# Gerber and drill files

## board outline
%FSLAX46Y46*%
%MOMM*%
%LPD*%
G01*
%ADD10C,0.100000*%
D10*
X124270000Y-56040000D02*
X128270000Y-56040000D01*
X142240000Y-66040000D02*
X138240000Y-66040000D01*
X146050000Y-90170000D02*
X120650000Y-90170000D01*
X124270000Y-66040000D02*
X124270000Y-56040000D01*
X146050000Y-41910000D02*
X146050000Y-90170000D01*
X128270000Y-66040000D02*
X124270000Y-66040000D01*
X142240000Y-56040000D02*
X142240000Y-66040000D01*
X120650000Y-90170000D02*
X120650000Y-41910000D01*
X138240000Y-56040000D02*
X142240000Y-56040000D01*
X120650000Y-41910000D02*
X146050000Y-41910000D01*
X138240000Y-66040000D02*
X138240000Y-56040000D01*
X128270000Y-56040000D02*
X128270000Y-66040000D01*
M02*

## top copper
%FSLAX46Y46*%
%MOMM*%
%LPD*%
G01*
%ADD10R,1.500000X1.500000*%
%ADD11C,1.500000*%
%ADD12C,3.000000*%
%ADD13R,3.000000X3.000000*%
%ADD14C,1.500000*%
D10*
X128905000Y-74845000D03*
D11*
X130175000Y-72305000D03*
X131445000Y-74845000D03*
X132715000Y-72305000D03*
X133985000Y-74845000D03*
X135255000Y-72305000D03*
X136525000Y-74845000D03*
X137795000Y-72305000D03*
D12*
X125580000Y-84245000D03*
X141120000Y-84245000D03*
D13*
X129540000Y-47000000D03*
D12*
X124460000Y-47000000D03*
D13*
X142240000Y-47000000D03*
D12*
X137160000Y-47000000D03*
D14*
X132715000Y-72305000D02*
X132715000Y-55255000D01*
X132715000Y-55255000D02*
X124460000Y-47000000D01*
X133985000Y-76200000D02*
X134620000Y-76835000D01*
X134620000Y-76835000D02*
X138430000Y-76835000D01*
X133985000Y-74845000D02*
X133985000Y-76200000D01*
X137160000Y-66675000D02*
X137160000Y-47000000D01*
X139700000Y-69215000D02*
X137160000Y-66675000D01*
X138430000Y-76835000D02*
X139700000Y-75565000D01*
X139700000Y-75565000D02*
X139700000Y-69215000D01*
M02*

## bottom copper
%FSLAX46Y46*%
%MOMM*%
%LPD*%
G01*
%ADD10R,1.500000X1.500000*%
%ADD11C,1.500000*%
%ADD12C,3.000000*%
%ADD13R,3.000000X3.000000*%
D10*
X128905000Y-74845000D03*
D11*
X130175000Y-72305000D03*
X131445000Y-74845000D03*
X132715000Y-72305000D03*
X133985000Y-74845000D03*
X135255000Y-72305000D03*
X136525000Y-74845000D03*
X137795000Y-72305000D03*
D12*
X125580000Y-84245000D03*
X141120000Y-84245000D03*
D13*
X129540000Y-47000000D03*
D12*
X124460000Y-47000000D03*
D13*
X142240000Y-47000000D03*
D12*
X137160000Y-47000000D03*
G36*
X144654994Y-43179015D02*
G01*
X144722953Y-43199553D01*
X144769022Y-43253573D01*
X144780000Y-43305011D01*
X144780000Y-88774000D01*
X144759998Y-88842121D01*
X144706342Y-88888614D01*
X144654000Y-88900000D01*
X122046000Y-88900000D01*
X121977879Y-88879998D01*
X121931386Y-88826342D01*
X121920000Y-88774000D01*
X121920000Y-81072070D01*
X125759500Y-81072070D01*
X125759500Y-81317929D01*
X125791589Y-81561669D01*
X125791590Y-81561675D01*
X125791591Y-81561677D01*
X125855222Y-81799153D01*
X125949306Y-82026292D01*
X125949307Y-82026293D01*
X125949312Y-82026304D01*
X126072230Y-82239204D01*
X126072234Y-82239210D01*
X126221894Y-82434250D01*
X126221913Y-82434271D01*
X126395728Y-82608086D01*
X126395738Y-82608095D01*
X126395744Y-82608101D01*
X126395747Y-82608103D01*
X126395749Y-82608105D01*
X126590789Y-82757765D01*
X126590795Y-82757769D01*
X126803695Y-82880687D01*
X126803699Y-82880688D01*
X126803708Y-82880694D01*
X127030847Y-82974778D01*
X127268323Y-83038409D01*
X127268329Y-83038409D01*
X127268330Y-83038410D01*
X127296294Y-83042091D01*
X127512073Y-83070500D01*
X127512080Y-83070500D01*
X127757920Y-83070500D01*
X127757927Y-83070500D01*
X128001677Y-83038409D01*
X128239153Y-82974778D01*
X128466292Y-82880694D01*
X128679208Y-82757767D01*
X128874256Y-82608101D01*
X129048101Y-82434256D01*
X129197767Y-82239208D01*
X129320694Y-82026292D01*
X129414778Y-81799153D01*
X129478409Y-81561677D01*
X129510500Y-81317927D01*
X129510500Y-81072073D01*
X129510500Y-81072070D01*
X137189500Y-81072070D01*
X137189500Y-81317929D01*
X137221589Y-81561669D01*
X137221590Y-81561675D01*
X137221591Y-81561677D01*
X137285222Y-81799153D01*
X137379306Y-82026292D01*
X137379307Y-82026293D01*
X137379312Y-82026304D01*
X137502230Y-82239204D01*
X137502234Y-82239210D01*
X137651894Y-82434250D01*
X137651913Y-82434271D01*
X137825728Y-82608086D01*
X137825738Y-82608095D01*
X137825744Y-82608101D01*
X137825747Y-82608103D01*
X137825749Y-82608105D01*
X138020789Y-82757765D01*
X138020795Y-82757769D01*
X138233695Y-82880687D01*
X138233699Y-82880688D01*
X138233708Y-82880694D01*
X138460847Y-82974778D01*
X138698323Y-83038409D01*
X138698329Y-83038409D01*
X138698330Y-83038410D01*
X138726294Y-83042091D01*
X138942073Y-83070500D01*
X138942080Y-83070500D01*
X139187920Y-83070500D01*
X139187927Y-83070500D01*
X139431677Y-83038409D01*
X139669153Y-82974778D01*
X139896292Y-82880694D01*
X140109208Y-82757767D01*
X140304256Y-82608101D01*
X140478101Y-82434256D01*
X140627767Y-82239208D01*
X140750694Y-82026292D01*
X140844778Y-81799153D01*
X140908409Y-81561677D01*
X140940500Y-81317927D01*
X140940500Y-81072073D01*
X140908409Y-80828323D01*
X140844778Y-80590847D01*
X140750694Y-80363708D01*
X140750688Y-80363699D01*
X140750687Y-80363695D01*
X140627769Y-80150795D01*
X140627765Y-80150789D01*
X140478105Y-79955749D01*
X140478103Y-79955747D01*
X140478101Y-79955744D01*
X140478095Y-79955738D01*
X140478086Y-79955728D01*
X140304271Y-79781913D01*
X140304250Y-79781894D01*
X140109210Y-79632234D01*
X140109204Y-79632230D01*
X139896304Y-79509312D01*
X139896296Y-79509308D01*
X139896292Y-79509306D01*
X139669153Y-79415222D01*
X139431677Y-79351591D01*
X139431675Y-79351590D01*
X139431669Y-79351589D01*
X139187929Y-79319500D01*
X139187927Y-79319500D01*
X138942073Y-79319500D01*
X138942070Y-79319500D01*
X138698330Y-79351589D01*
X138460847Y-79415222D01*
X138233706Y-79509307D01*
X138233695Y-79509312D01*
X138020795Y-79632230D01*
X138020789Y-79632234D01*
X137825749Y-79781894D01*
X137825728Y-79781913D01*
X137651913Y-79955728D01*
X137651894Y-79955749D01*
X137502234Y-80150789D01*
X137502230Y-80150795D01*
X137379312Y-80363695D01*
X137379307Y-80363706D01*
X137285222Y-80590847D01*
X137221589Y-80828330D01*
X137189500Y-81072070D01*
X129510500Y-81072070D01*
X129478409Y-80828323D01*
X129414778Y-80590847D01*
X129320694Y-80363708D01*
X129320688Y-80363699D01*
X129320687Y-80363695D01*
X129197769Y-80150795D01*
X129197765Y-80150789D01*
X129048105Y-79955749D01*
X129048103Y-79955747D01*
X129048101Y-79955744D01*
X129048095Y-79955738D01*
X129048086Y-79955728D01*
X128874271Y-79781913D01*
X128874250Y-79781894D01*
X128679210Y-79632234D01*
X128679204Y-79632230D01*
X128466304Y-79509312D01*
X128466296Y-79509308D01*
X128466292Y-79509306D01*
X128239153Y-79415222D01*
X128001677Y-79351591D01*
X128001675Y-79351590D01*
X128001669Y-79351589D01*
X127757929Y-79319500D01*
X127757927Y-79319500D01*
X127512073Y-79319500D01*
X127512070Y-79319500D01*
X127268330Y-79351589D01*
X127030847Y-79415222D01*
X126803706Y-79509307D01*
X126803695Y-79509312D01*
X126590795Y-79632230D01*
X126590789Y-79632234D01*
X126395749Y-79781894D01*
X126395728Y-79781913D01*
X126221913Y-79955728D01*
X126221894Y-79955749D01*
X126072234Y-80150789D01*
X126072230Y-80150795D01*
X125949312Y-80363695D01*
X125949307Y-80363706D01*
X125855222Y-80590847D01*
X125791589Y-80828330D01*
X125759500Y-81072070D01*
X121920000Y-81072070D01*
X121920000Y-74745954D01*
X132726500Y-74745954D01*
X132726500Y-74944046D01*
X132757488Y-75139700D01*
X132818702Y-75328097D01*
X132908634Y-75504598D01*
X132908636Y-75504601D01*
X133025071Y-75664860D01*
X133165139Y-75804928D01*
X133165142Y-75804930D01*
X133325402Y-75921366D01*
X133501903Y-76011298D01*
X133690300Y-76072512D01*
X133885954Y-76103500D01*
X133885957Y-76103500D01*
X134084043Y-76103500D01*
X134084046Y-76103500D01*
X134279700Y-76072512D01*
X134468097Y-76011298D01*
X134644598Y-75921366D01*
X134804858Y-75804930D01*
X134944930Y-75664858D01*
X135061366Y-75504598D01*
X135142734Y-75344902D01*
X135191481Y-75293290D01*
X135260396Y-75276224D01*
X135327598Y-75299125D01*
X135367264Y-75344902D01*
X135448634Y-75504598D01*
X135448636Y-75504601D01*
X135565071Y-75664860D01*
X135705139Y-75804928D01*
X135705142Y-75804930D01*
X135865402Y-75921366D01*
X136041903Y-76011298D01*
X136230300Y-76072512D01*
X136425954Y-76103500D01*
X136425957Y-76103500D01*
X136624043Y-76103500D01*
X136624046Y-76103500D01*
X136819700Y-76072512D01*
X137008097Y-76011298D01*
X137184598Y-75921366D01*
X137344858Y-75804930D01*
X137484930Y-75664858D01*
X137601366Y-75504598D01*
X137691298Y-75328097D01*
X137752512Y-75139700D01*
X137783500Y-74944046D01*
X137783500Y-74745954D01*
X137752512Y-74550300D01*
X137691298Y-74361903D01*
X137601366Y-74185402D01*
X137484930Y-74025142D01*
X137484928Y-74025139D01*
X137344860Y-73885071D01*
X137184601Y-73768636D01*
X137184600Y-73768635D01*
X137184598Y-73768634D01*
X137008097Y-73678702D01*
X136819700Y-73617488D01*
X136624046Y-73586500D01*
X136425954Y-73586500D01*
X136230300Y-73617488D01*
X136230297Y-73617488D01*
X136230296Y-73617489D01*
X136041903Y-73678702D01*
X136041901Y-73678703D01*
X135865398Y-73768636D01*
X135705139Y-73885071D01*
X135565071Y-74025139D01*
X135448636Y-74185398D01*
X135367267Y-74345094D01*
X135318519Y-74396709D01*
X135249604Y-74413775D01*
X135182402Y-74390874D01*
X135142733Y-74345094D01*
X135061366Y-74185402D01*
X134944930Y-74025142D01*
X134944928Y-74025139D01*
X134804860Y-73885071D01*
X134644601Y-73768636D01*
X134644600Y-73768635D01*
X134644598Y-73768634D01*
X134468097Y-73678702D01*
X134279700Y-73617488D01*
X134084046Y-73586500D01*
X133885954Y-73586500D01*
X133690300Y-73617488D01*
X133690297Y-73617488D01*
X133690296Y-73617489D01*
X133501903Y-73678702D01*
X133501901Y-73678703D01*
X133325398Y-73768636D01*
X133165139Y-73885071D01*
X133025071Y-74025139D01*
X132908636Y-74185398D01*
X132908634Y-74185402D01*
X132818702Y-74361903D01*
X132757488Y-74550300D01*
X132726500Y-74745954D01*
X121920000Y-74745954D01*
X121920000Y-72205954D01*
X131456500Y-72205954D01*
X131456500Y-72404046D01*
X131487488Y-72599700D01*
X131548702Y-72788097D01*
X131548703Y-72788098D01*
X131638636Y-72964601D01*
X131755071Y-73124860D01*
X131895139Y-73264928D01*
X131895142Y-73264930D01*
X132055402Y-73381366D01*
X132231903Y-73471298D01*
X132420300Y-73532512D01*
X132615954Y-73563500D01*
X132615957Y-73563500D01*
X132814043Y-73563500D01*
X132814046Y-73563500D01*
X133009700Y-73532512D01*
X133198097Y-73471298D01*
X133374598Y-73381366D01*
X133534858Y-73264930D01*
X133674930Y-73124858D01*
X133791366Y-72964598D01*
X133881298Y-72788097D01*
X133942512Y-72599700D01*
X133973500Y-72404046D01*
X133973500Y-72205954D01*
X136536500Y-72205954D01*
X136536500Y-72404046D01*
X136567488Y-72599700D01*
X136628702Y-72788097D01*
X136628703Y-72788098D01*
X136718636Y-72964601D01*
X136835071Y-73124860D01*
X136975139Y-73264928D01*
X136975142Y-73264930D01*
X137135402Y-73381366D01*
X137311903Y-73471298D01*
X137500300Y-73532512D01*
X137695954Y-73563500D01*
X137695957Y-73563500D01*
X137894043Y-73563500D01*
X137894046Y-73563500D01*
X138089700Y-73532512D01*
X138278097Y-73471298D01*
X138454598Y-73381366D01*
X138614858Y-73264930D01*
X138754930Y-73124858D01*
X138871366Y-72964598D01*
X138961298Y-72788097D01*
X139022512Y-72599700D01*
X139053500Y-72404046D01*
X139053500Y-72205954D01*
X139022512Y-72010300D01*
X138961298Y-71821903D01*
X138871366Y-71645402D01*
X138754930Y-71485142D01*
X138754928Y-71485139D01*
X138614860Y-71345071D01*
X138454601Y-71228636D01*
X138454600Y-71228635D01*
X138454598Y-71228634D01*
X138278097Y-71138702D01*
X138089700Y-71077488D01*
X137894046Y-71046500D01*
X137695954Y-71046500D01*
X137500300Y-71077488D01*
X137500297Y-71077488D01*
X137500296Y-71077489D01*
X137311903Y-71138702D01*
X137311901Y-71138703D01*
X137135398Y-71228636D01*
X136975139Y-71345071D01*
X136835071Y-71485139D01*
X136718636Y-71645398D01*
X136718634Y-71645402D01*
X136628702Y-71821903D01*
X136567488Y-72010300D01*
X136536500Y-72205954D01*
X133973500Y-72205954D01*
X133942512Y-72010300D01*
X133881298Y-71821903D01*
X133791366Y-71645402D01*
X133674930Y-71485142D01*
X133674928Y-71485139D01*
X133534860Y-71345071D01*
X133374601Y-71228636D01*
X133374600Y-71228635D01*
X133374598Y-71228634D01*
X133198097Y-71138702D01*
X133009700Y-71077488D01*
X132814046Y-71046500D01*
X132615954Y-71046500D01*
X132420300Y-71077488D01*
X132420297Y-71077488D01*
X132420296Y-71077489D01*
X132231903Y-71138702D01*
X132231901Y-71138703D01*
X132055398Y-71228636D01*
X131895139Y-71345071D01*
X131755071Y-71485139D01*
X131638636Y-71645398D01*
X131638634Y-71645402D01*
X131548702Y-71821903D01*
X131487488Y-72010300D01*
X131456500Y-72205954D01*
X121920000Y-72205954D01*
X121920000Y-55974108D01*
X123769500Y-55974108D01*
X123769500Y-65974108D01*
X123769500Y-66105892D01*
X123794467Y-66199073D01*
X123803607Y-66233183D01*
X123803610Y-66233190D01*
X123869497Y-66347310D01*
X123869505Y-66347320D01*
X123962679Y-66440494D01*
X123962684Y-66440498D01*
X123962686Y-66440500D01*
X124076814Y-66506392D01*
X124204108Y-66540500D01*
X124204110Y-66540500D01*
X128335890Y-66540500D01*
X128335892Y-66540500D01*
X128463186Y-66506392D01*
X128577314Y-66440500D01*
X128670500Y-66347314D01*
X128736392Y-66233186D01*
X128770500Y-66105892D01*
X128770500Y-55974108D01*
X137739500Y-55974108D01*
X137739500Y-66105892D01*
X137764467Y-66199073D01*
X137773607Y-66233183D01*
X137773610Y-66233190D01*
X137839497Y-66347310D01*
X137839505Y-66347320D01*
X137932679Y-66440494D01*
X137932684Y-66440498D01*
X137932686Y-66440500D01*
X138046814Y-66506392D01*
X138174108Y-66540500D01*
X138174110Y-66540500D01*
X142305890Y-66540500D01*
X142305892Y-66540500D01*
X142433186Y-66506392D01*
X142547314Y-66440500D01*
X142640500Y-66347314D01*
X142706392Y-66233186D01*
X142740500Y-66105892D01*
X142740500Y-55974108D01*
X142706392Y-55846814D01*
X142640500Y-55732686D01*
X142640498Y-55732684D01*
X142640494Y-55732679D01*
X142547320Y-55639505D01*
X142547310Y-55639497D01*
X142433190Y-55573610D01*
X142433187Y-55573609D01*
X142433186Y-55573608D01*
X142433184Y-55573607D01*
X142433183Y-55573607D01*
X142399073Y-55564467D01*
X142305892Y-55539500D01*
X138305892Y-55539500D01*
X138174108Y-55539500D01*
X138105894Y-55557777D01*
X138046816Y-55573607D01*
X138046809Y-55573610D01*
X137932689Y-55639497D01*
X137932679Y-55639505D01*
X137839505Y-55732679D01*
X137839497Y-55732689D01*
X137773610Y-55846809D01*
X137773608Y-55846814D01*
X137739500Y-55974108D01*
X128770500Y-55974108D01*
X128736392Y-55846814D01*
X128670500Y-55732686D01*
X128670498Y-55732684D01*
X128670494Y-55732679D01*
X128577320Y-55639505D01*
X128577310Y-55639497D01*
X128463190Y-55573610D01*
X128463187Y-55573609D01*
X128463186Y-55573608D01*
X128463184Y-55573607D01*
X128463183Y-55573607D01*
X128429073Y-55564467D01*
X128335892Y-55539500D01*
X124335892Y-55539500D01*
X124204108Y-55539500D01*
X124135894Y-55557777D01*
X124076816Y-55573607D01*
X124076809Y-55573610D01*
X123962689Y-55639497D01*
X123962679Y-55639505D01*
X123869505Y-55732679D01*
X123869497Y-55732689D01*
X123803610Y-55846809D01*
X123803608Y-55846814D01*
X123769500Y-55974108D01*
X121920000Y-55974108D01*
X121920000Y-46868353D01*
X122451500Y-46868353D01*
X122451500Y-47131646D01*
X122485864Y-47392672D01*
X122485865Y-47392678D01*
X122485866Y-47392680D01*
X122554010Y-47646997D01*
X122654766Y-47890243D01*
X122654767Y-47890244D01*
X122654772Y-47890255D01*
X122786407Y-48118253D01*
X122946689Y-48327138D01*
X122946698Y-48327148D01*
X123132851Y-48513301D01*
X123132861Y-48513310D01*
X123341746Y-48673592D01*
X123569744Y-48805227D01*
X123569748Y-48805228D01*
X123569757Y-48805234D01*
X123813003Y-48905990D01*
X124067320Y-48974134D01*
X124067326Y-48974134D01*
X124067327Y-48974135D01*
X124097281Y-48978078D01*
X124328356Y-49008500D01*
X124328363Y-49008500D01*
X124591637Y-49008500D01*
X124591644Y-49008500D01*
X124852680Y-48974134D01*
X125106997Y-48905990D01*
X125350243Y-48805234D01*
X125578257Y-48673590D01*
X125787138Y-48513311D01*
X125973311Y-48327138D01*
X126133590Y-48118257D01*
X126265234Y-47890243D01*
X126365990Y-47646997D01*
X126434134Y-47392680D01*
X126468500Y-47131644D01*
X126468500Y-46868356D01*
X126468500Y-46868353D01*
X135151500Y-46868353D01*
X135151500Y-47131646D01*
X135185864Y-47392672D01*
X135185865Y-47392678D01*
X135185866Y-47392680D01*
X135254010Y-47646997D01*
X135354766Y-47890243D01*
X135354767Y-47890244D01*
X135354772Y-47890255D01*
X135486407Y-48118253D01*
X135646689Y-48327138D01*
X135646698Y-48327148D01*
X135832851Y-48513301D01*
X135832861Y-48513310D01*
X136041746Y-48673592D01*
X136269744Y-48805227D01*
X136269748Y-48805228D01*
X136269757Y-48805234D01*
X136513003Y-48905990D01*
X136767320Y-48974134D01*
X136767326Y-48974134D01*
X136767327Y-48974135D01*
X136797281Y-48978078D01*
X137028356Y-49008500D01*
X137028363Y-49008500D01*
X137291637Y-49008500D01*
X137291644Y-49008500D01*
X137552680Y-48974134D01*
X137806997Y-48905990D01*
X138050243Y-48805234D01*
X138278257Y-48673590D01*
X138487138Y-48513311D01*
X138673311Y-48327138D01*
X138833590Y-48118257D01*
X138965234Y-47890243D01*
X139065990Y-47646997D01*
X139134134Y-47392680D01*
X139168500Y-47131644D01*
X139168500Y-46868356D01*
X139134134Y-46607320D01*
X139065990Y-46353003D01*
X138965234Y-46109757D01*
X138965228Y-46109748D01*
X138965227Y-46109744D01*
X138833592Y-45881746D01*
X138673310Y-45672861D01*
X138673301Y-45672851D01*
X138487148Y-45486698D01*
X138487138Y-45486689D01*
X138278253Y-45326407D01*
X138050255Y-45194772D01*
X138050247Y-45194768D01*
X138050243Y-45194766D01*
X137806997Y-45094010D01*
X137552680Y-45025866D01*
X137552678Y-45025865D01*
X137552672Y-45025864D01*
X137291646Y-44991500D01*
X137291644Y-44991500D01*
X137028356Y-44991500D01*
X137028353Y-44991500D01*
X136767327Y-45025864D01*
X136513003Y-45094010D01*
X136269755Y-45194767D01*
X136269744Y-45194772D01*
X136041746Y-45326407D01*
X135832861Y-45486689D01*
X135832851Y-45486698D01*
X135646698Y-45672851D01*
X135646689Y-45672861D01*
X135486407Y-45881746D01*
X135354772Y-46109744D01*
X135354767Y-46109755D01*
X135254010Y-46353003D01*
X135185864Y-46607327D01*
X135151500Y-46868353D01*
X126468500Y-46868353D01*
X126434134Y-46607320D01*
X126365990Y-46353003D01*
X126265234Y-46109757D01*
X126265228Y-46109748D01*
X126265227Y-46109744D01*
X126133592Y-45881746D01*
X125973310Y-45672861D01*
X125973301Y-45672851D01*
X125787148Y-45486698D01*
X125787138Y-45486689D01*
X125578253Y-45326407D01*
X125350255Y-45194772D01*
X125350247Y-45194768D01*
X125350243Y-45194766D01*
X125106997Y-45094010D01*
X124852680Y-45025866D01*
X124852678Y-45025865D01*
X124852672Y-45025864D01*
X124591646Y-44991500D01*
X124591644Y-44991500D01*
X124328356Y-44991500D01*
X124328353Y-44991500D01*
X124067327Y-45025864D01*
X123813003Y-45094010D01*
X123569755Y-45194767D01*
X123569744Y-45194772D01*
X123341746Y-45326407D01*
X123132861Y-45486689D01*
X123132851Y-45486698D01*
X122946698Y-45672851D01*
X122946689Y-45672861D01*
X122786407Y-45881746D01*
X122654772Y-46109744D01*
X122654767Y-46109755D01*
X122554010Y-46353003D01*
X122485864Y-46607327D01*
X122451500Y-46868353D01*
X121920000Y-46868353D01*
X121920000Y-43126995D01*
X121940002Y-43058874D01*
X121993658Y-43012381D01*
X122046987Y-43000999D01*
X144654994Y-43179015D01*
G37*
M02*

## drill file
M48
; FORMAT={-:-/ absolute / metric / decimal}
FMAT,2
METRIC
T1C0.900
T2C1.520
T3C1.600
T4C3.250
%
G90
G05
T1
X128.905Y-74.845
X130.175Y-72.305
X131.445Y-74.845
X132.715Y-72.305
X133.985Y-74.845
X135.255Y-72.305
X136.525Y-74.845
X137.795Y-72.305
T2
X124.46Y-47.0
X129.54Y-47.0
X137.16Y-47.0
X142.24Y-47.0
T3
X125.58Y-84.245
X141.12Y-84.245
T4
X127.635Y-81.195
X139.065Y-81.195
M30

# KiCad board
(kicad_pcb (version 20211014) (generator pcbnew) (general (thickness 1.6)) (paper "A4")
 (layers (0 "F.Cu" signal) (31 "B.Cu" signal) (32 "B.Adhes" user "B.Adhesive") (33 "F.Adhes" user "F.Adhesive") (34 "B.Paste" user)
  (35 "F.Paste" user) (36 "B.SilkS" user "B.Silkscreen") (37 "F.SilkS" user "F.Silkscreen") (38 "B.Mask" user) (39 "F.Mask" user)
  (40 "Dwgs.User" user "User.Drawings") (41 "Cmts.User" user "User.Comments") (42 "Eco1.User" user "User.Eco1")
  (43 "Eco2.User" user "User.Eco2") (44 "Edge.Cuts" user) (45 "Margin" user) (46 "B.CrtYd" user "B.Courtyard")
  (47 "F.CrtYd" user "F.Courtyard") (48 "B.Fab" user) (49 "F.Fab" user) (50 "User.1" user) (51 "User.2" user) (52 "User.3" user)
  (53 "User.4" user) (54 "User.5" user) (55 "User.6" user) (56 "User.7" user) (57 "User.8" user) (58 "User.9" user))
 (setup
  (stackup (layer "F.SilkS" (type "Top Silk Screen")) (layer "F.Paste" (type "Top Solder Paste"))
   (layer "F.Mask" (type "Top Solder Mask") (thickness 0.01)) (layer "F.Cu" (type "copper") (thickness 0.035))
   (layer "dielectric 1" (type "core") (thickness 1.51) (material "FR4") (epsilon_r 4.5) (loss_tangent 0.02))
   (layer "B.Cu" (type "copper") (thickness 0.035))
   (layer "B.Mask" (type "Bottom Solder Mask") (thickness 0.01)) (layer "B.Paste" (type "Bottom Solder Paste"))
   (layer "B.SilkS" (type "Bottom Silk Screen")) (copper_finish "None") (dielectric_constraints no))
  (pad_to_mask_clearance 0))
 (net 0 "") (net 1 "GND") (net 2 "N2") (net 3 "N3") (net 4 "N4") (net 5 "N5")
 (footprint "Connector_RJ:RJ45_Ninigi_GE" (layer "F.Cu") (at 128.905 74.845)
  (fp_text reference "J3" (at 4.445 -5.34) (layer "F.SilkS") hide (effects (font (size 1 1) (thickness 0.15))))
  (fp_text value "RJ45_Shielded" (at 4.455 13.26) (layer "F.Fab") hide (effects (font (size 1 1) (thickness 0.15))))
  (pad "" np_thru_hole circle (at -1.27 6.35) (size 3.25 3.25) (drill 3.25) (layers *.Cu *.Mask))
  (pad "" np_thru_hole circle (at 10.16 6.35 180) (size 3.25 3.25) (drill 3.25) (layers *.Cu *.Mask))
  (pad "1" thru_hole rect (at 0 0 180) (size 1.5 1.5) (drill 0.9) (layers *.Cu *.Mask) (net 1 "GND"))
  (pad "2" thru_hole circle (at 1.27 -2.54 180) (size 1.5 1.5) (drill 0.9) (layers *.Cu *.Mask) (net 1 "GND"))
  (pad "3" thru_hole circle (at 2.54 0 180) (size 1.5 1.5) (drill 0.9) (layers *.Cu *.Mask) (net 1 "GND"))
  (pad "4" thru_hole circle (at 3.81 -2.54 180) (size 1.5 1.5) (drill 0.9) (layers *.Cu *.Mask) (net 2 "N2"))
  (pad "5" thru_hole circle (at 5.08 0 180) (size 1.5 1.5) (drill 0.9) (layers *.Cu *.Mask) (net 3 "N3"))
  (pad "6" thru_hole circle (at 6.35 -2.54 180) (size 1.5 1.5) (drill 0.9) (layers *.Cu *.Mask) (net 1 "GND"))
  (pad "7" thru_hole circle (at 7.62 0 180) (size 1.5 1.5) (drill 0.9) (layers *.Cu *.Mask) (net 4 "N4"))
  (pad "8" thru_hole circle (at 8.89 -2.54 180) (size 1.5 1.5) (drill 0.9) (layers *.Cu *.Mask) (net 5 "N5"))
  (pad "SH" thru_hole circle (at -3.325 9.4) (size 3 3) (drill 1.6) (layers *.Cu *.Mask) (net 1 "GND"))
  (pad "SH" thru_hole circle (at 12.215 9.4 180) (size 3 3) (drill 1.6) (layers *.Cu *.Mask) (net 1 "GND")))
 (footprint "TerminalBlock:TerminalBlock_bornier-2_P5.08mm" (layer "F.Cu") (at 129.54 47 180)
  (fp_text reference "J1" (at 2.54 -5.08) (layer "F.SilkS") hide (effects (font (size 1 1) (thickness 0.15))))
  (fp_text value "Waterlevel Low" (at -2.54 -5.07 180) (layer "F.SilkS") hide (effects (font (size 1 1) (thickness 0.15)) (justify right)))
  (pad "1" thru_hole rect (at 0 0 180) (size 3 3) (drill 1.52) (layers *.Cu *.Mask) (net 1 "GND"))
  (pad "2" thru_hole circle (at 5.08 0 180) (size 3 3) (drill 1.52) (layers *.Cu *.Mask) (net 2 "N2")))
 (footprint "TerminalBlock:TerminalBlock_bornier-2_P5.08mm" (layer "F.Cu") (at 142.24 47 180)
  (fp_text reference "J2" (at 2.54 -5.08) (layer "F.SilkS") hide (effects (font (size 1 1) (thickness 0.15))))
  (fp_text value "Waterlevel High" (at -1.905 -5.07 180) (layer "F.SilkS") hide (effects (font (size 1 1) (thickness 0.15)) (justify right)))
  (pad "1" thru_hole rect (at 0 0 180) (size 3 3) (drill 1.52) (layers *.Cu *.Mask) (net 1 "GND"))
  (pad "2" thru_hole circle (at 5.08 0 180) (size 3 3) (drill 1.52) (layers *.Cu *.Mask) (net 3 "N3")))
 (gr_line (start 124.27 56.04) (end 128.27 56.04) (layer "Edge.Cuts") (width 0.1))
 (gr_line (start 142.24 66.04) (end 138.24 66.04) (layer "Edge.Cuts") (width 0.1))
 (gr_line (start 146.05 90.17) (end 120.65 90.17) (layer "Edge.Cuts") (width 0.1))
 (gr_line (start 124.27 66.04) (end 124.27 56.04) (layer "Edge.Cuts") (width 0.1))
 (gr_line (start 146.05 41.91) (end 146.05 90.17) (layer "Edge.Cuts") (width 0.1))
 (gr_line (start 128.27 66.04) (end 124.27 66.04) (layer "Edge.Cuts") (width 0.1))
 (gr_line (start 142.24 56.04) (end 142.24 66.04) (layer "Edge.Cuts") (width 0.1))
 (gr_line (start 120.65 90.17) (end 120.65 41.91) (layer "Edge.Cuts") (width 0.1))
 (gr_line (start 138.24 56.04) (end 142.24 56.04) (layer "Edge.Cuts") (width 0.1))
 (gr_line (start 120.65 41.91) (end 146.05 41.91) (layer "Edge.Cuts") (width 0.1))
 (gr_line (start 138.24 66.04) (end 138.24 56.04) (layer "Edge.Cuts") (width 0.1))
 (gr_line (start 128.27 56.04) (end 128.27 66.04) (layer "Edge.Cuts") (width 0.1))
 (segment (start 132.715 72.305) (end 132.715 55.255) (width 1.5) (layer "F.Cu") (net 2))
 (segment (start 132.715 55.255) (end 124.46 47) (width 1.5) (layer "F.Cu") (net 2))
 (segment (start 133.985 76.2) (end 134.62 76.835) (width 1.5) (layer "F.Cu") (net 3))
 (segment (start 134.62 76.835) (end 138.43 76.835) (width 1.5) (layer "F.Cu") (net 3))
 (segment (start 133.985 74.845) (end 133.985 76.2) (width 1.5) (layer "F.Cu") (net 3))
 (segment (start 137.16 66.675) (end 137.16 47) (width 1.5) (layer "F.Cu") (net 3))
 (segment (start 139.7 69.215) (end 137.16 66.675) (width 1.5) (layer "F.Cu") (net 3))
 (segment (start 138.43 76.835) (end 139.7 75.565) (width 1.5) (layer "F.Cu") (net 3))
 (segment (start 139.7 75.565) (end 139.7 69.215) (width 1.5) (layer "F.Cu") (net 3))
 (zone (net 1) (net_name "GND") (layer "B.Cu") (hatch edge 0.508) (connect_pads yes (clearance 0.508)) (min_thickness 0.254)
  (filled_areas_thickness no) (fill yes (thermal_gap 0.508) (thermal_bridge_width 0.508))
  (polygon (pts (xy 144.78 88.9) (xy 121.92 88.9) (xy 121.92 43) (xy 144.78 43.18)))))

